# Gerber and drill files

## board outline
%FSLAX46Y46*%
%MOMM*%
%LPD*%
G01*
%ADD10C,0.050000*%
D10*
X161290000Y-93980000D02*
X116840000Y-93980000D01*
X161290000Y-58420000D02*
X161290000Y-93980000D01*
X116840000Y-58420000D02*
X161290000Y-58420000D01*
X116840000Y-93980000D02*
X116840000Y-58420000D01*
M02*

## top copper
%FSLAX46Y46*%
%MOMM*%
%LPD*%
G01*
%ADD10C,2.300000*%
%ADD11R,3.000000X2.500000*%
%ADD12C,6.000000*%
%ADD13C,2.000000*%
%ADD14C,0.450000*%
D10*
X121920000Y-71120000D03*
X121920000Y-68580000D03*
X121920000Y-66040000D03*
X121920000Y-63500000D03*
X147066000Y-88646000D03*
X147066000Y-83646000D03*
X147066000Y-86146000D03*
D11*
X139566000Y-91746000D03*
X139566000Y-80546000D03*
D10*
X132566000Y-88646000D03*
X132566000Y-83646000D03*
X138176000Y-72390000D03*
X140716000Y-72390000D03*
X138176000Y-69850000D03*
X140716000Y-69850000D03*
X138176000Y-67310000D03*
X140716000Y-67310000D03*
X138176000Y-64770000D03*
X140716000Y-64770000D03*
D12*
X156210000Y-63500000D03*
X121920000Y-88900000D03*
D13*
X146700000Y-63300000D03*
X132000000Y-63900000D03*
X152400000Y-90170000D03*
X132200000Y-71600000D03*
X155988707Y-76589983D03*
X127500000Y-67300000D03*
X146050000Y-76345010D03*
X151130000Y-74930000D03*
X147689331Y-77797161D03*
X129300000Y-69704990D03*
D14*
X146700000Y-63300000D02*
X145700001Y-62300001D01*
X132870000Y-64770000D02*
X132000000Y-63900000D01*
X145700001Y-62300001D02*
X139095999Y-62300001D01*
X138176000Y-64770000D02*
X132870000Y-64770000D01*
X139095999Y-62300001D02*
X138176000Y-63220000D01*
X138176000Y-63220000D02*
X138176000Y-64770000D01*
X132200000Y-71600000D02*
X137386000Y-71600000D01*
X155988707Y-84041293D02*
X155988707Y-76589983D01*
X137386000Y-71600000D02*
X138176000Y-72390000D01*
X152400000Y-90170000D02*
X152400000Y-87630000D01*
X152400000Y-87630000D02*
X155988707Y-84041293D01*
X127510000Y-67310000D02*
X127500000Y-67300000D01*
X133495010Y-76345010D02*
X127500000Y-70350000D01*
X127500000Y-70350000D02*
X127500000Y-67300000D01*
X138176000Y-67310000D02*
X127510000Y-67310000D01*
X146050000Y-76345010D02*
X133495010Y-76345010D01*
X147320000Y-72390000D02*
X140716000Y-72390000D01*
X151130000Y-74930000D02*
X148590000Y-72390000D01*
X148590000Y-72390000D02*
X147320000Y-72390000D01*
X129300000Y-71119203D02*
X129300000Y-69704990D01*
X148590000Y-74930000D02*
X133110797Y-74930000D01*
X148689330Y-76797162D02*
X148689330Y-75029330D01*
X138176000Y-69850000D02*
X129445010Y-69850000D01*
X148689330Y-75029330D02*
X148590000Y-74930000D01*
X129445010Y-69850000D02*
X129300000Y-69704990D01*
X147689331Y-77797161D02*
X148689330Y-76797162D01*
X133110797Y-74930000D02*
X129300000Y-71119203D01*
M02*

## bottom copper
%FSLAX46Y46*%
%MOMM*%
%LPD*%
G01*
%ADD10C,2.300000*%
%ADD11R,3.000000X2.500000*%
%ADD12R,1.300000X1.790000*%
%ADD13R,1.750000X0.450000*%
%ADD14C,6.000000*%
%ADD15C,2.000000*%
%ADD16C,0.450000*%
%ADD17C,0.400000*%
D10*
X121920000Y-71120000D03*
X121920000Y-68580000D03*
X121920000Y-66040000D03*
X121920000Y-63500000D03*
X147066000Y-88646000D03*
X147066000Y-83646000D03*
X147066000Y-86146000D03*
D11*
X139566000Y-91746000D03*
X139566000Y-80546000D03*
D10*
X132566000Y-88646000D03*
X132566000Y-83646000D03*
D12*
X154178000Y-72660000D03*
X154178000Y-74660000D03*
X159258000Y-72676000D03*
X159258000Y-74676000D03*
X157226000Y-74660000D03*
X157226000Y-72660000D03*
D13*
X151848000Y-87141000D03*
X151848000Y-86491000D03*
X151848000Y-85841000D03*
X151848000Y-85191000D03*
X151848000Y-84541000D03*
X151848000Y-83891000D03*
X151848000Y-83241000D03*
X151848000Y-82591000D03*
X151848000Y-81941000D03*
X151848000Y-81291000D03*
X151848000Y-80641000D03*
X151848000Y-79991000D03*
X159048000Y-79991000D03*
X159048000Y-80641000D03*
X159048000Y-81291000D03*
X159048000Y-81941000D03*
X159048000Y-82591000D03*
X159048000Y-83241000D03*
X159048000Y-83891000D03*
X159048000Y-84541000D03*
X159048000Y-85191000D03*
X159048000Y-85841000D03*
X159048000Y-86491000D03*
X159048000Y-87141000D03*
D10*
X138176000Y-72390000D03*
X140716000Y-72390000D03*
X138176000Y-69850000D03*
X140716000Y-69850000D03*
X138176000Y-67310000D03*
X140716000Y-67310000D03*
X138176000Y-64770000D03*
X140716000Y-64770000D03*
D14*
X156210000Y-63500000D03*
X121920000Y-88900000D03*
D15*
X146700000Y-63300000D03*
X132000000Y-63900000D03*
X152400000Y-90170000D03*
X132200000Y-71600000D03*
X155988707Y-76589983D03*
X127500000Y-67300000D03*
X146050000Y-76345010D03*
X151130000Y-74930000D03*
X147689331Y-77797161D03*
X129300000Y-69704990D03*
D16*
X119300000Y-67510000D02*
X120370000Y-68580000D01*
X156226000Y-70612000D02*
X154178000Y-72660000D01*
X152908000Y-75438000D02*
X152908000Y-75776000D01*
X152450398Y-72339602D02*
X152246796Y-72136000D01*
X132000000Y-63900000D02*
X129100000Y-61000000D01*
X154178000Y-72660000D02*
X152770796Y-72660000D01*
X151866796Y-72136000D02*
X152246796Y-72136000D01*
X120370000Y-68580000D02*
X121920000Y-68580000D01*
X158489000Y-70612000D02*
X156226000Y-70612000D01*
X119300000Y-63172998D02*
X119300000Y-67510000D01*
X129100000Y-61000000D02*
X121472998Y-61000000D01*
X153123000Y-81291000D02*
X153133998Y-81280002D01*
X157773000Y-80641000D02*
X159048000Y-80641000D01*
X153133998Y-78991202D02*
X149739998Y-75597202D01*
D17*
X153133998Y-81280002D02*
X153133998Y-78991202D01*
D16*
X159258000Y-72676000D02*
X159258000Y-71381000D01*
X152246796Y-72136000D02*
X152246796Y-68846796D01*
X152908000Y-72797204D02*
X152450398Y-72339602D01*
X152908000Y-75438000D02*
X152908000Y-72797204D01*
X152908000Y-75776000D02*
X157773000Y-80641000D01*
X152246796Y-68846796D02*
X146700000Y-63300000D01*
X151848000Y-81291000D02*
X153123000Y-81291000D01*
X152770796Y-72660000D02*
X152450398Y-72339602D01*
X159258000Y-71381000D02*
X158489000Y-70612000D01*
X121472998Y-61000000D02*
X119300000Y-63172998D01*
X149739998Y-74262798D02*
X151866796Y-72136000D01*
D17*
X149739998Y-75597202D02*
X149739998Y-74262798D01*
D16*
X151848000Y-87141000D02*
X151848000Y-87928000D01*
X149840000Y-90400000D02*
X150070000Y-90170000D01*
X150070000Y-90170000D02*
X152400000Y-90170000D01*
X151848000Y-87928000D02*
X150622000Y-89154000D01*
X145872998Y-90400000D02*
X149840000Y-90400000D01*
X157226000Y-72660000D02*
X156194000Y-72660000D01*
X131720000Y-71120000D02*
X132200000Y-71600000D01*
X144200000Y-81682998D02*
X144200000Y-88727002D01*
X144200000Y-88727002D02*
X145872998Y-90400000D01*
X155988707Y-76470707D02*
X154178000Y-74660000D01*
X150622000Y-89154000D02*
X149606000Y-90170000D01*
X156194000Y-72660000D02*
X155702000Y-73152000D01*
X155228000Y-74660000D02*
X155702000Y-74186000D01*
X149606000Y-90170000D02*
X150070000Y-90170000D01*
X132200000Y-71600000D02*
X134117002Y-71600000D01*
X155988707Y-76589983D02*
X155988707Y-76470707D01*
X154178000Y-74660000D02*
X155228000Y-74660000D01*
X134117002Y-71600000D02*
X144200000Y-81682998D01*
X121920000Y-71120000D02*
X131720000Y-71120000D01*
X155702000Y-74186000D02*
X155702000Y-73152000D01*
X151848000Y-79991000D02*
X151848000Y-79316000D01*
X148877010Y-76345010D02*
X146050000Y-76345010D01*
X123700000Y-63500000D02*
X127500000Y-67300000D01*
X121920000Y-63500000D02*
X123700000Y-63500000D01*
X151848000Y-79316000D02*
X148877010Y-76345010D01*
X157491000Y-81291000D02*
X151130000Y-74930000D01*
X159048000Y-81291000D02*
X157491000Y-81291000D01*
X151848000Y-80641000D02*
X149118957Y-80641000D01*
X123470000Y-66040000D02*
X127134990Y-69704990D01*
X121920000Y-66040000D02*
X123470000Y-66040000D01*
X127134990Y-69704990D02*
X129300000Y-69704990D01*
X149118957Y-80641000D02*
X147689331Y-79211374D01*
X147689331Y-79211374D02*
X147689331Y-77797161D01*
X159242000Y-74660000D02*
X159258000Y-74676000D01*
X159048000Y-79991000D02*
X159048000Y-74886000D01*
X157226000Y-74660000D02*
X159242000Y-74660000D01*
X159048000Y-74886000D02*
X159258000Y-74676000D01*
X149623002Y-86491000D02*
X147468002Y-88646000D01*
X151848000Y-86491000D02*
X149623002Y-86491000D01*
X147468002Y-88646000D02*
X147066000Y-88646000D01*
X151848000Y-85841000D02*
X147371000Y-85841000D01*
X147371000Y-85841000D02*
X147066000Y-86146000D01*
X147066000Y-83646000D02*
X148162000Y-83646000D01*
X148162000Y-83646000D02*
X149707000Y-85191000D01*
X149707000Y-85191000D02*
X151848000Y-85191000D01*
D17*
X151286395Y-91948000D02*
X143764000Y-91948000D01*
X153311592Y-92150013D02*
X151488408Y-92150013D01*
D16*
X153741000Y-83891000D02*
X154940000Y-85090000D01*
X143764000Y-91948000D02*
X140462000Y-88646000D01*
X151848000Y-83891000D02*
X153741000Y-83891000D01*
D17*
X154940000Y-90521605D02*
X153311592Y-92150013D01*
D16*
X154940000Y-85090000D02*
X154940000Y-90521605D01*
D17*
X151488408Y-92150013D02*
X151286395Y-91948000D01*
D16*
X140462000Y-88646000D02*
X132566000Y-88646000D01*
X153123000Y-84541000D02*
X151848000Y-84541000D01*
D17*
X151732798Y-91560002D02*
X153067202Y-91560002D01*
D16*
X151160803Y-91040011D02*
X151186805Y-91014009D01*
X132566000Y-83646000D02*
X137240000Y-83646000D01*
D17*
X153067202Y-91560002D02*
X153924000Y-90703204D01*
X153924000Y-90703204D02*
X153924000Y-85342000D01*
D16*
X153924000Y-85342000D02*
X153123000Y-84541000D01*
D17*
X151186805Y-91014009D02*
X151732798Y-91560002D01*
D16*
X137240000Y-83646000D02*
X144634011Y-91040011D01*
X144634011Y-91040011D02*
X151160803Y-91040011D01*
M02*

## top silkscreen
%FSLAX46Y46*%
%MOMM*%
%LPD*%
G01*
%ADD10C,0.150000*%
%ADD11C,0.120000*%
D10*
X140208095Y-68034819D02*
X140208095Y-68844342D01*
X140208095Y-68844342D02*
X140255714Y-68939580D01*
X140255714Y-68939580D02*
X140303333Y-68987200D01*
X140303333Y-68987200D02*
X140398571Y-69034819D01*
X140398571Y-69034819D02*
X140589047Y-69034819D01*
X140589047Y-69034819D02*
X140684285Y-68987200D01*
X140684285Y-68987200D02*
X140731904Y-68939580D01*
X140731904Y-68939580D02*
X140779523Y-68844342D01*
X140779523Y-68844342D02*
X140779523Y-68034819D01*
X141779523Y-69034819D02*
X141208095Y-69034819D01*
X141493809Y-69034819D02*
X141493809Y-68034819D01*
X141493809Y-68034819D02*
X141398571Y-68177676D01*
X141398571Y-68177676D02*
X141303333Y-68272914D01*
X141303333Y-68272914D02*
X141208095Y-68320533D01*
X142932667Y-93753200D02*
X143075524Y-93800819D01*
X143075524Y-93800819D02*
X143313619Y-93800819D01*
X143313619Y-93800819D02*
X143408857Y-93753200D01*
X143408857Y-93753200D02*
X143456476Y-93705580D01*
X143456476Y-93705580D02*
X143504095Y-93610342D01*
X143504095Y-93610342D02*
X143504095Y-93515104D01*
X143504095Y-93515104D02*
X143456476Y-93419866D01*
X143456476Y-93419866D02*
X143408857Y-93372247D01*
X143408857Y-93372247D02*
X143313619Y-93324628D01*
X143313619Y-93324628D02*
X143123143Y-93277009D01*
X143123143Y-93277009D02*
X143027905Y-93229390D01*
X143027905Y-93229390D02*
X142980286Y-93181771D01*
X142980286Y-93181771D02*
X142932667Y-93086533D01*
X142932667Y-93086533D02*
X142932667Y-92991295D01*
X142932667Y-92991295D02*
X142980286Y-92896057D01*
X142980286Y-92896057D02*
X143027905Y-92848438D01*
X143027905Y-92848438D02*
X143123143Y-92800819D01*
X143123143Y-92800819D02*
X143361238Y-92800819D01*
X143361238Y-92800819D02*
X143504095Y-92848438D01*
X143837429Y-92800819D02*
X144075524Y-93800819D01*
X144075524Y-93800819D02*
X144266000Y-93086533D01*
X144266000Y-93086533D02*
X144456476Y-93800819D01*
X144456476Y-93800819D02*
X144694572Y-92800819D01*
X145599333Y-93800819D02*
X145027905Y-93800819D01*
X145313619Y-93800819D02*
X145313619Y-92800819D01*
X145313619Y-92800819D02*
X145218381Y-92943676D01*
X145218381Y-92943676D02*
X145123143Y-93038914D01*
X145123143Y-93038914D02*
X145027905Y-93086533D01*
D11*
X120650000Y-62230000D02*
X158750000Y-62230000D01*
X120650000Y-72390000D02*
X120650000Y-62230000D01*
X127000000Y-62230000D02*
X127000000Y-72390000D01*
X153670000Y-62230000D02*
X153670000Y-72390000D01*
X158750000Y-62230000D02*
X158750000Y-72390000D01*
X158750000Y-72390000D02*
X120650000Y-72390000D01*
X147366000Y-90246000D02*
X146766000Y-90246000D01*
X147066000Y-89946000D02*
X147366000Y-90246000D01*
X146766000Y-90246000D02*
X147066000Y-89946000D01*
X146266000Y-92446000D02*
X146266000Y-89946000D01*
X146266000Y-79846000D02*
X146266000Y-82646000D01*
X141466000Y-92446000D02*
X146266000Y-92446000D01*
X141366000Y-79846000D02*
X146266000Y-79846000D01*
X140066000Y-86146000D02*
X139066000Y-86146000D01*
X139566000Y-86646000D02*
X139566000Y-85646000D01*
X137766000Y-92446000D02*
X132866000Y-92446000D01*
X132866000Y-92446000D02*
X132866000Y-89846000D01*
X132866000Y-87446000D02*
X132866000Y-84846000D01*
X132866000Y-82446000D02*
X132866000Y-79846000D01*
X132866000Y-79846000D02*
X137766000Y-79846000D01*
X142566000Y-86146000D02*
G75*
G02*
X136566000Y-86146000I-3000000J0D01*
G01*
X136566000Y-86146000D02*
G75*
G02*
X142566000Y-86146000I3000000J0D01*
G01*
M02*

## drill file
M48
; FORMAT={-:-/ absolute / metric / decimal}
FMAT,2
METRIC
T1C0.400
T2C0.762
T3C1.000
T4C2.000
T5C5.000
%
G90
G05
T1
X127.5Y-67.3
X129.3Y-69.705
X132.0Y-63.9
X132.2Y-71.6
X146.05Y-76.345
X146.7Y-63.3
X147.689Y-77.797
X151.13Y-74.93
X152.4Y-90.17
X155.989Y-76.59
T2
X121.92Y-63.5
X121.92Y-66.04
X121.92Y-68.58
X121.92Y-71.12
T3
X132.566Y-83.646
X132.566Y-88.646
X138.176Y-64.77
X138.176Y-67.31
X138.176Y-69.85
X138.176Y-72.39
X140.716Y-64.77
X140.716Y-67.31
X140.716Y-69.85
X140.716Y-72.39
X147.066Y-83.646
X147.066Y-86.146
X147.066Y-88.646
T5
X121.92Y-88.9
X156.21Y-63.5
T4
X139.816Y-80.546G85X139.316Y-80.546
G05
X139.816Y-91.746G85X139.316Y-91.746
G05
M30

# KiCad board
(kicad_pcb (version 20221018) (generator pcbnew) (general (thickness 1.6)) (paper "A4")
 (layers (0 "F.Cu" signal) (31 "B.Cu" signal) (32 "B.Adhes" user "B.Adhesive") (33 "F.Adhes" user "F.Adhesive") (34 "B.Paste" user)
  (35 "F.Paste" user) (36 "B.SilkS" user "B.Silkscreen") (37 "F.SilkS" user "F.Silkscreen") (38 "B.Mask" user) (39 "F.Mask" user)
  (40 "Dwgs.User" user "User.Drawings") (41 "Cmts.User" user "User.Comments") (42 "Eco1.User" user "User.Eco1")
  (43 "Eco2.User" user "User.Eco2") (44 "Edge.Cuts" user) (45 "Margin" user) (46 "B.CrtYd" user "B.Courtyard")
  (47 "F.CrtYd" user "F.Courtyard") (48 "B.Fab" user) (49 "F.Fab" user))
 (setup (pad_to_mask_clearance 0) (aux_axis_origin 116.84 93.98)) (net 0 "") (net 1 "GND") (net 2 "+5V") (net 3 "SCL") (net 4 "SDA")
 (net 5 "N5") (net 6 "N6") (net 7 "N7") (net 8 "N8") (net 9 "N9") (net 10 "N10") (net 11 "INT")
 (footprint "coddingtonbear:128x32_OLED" (layer "F.Cu") (at 129.54 68.58)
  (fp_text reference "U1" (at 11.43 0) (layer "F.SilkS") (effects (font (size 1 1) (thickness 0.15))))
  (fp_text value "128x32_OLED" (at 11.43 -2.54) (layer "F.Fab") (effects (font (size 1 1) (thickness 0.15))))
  (fp_line (start -8.89 -6.35) (end 29.21 -6.35) (stroke (width 0.12) (type solid)) (layer "F.SilkS"))
  (fp_line (start -8.89 3.81) (end -8.89 -6.35) (stroke (width 0.12) (type solid)) (layer "F.SilkS"))
  (fp_line (start -2.54 -6.35) (end -2.54 3.81) (stroke (width 0.12) (type solid)) (layer "F.SilkS"))
  (fp_line (start 24.13 -6.35) (end 24.13 3.81) (stroke (width 0.12) (type solid)) (layer "F.SilkS"))
  (fp_line (start 29.21 -6.35) (end 29.21 3.81) (stroke (width 0.12) (type solid)) (layer "F.SilkS"))
  (fp_line (start 29.21 3.81) (end -8.89 3.81) (stroke (width 0.12) (type solid)) (layer "F.SilkS"))
  (pad "1" thru_hole circle (at -7.62 2.54) (size 2.3 2.3) (drill 0.762) (layers "*.Cu" "*.Mask") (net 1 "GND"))
  (pad "2" thru_hole circle (at -7.62 0) (size 2.3 2.3) (drill 0.762) (layers "*.Cu" "*.Mask") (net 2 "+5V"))
  (pad "3" thru_hole circle (at -7.62 -2.54) (size 2.3 2.3) (drill 0.762) (layers "*.Cu" "*.Mask") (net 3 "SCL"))
  (pad "4" thru_hole circle (at -7.62 -5.08) (size 2.3 2.3) (drill 0.762) (layers "*.Cu" "*.Mask") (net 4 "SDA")))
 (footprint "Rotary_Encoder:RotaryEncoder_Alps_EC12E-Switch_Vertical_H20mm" (layer "F.Cu") (at 147.066 88.646 180)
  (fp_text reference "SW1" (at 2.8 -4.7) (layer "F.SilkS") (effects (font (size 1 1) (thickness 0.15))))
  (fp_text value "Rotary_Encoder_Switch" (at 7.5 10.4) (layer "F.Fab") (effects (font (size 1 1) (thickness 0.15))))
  (fp_line (start -0.3 -1.6) (end 0.3 -1.6) (stroke (width 0.12) (type solid)) (layer "F.SilkS"))
  (fp_line (start 0 -1.3) (end -0.3 -1.6) (stroke (width 0.12) (type solid)) (layer "F.SilkS"))
  (fp_line (start 0.3 -1.6) (end 0 -1.3) (stroke (width 0.12) (type solid)) (layer "F.SilkS"))
  (fp_line (start 0.8 -3.8) (end 0.8 -1.3) (stroke (width 0.12) (type solid)) (layer "F.SilkS"))
  (fp_line (start 0.8 8.8) (end 0.8 6) (stroke (width 0.12) (type solid)) (layer "F.SilkS"))
  (fp_line (start 5.6 -3.8) (end 0.8 -3.8) (stroke (width 0.12) (type solid)) (layer "F.SilkS"))
  (fp_line (start 5.7 8.8) (end 0.8 8.8) (stroke (width 0.12) (type solid)) (layer "F.SilkS"))
  (fp_line (start 7 2.5) (end 8 2.5) (stroke (width 0.12) (type solid)) (layer "F.SilkS"))
  (fp_line (start 7.5 2) (end 7.5 3) (stroke (width 0.12) (type solid)) (layer "F.SilkS"))
  (fp_line (start 9.3 -3.8) (end 14.2 -3.8) (stroke (width 0.12) (type solid)) (layer "F.SilkS"))
  (fp_line (start 14.2 -3.8) (end 14.2 -1.2) (stroke (width 0.12) (type solid)) (layer "F.SilkS"))
  (fp_line (start 14.2 1.2) (end 14.2 3.8) (stroke (width 0.12) (type solid)) (layer "F.SilkS"))
  (fp_line (start 14.2 6.2) (end 14.2 8.8) (stroke (width 0.12) (type solid)) (layer "F.SilkS"))
  (fp_line (start 14.2 8.8) (end 9.3 8.8) (stroke (width 0.12) (type solid)) (layer "F.SilkS"))
  (fp_circle (center 7.5 2.5) (end 10.5 2.5) (stroke (width 0.12) (type solid)) (fill none) (layer "F.SilkS"))
  (pad "A" thru_hole circle (at 0 0 180) (size 2.3 2.3) (drill 1) (layers "*.Cu" "*.Mask") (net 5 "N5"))
  (pad "B" thru_hole circle (at 0 5 180) (size 2.3 2.3) (drill 1) (layers "*.Cu" "*.Mask") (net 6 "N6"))
  (pad "C" thru_hole circle (at 0 2.5 180) (size 2.3 2.3) (drill 1) (layers "*.Cu" "*.Mask") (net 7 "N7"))
  (pad "MP" thru_hole rect (at 7.5 -3.1 180) (size 3 2.5) (drill oval 2.5 2) (layers "*.Cu" "*.Mask"))
  (pad "MP" thru_hole rect (at 7.5 8.1 180) (size 3 2.5) (drill oval 2.5 2) (layers "*.Cu" "*.Mask"))
  (pad "S1" thru_hole circle (at 14.5 0 180) (size 2.3 2.3) (drill 1) (layers "*.Cu" "*.Mask") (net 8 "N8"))
  (pad "S2" thru_hole circle (at 14.5 5 180) (size 2.3 2.3) (drill 1) (layers "*.Cu" "*.Mask") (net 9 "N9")))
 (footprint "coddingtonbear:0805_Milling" (layer "B.Cu") (at 154.178 73.66 -90)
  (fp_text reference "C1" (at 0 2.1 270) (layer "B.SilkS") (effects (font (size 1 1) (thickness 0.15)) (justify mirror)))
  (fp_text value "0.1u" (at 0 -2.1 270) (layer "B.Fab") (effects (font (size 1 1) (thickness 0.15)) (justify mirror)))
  (pad "1" smd rect (at -1 0 270) (size 1.79 1.3) (layers "B.Cu" "B.Paste" "B.Mask") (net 2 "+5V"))
  (pad "2" smd rect (at 1 0 270) (size 1.79 1.3) (layers "B.Cu" "B.Paste" "B.Mask") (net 1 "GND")))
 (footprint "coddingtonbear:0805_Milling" (layer "B.Cu") (at 159.258 73.676 -90)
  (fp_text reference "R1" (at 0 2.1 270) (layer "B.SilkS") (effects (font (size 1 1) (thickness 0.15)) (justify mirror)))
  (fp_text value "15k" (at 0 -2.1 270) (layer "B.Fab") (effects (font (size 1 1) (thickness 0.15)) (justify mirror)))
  (pad "1" smd rect (at -1 0 270) (size 1.79 1.3) (layers "B.Cu" "B.Paste" "B.Mask") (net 2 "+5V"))
  (pad "2" smd rect (at 1 0 270) (size 1.79 1.3) (layers "B.Cu" "B.Paste" "B.Mask") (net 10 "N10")))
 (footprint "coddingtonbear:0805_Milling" (layer "B.Cu") (at 157.226 73.66 90)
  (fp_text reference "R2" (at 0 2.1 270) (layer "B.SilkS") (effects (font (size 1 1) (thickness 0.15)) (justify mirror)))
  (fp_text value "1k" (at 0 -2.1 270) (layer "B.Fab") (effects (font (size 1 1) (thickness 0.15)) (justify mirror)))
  (pad "1" smd rect (at -1 0 90) (size 1.79 1.3) (layers "B.Cu" "B.Paste" "B.Mask") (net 10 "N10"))
  (pad "2" smd rect (at 1 0 90) (size 1.79 1.3) (layers "B.Cu" "B.Paste" "B.Mask") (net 1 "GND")))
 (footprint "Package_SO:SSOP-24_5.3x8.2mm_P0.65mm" (layer "B.Cu") (at 155.448 83.566)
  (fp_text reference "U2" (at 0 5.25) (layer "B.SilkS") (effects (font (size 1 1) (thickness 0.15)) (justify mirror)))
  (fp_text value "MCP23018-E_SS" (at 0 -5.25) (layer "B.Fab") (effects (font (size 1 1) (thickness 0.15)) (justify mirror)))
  (pad "1" smd rect (at -3.6 3.575) (size 1.75 0.45) (layers "B.Cu" "B.Paste" "B.Mask") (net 1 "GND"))
  (pad "2" smd rect (at -3.6 2.925) (size 1.75 0.45) (layers "B.Cu" "B.Paste" "B.Mask") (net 5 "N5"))
  (pad "3" smd rect (at -3.6 2.275) (size 1.75 0.45) (layers "B.Cu" "B.Paste" "B.Mask") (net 7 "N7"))
  (pad "4" smd rect (at -3.6 1.625) (size 1.75 0.45) (layers "B.Cu" "B.Paste" "B.Mask") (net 6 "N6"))
  (pad "5" smd rect (at -3.6 0.975) (size 1.75 0.45) (layers "B.Cu" "B.Paste" "B.Mask") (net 9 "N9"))
  (pad "6" smd rect (at -3.6 0.325) (size 1.75 0.45) (layers "B.Cu" "B.Paste" "B.Mask") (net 8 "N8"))
  (pad "7" smd rect (at -3.6 -0.325) (size 1.75 0.45) (layers "B.Cu" "B.Paste" "B.Mask"))
  (pad "8" smd rect (at -3.6 -0.975) (size 1.75 0.45) (layers "B.Cu" "B.Paste" "B.Mask"))
  (pad "9" smd rect (at -3.6 -1.625) (size 1.75 0.45) (layers "B.Cu" "B.Paste" "B.Mask"))
  (pad "10" smd rect (at -3.6 -2.275) (size 1.75 0.45) (layers "B.Cu" "B.Paste" "B.Mask") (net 2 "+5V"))
  (pad "11" smd rect (at -3.6 -2.925) (size 1.75 0.45) (layers "B.Cu" "B.Paste" "B.Mask") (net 3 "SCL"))
  (pad "12" smd rect (at -3.6 -3.575) (size 1.75 0.45) (layers "B.Cu" "B.Paste" "B.Mask") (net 4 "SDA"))
  (pad "13" smd rect (at 3.6 -3.575) (size 1.75 0.45) (layers "B.Cu" "B.Paste" "B.Mask") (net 10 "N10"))
  (pad "14" smd rect (at 3.6 -2.925) (size 1.75 0.45) (layers "B.Cu" "B.Paste" "B.Mask") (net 2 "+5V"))
  (pad "15" smd rect (at 3.6 -2.275) (size 1.75 0.45) (layers "B.Cu" "B.Paste" "B.Mask") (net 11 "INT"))
  (pad "16" smd rect (at 3.6 -1.625) (size 1.75 0.45) (layers "B.Cu" "B.Paste" "B.Mask"))
  (pad "17" smd rect (at 3.6 -0.975) (size 1.75 0.45) (layers "B.Cu" "B.Paste" "B.Mask"))
  (pad "18" smd rect (at 3.6 -0.325) (size 1.75 0.45) (layers "B.Cu" "B.Paste" "B.Mask"))
  (pad "19" smd rect (at 3.6 0.325) (size 1.75 0.45) (layers "B.Cu" "B.Paste" "B.Mask"))
  (pad "20" smd rect (at 3.6 0.975) (size 1.75 0.45) (layers "B.Cu" "B.Paste" "B.Mask"))
  (pad "21" smd rect (at 3.6 1.625) (size 1.75 0.45) (layers "B.Cu" "B.Paste" "B.Mask"))
  (pad "22" smd rect (at 3.6 2.275) (size 1.75 0.45) (layers "B.Cu" "B.Paste" "B.Mask"))
  (pad "23" smd rect (at 3.6 2.925) (size 1.75 0.45) (layers "B.Cu" "B.Paste" "B.Mask"))
  (pad "24" smd rect (at 3.6 3.575) (size 1.75 0.45) (layers "B.Cu" "B.Paste" "B.Mask")))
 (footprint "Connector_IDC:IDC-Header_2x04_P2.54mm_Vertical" (layer "B.Cu") (at 138.176 72.39)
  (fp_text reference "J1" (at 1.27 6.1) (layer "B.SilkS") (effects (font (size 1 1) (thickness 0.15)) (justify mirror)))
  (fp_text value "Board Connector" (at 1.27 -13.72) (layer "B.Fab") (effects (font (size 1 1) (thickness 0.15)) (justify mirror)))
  (pad "1" thru_hole circle (at 0 0) (size 2.3 2.3) (drill 1) (layers "*.Cu" "*.Mask") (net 1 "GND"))
  (pad "2" thru_hole circle (at 2.54 0) (size 2.3 2.3) (drill 1) (layers "*.Cu" "*.Mask") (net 11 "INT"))
  (pad "3" thru_hole circle (at 0 -2.54) (size 2.3 2.3) (drill 1) (layers "*.Cu" "*.Mask") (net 3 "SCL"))
  (pad "4" thru_hole circle (at 2.54 -2.54) (size 2.3 2.3) (drill 1) (layers "*.Cu" "*.Mask"))
  (pad "5" thru_hole circle (at 0 -5.08) (size 2.3 2.3) (drill 1) (layers "*.Cu" "*.Mask") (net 4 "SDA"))
  (pad "6" thru_hole circle (at 2.54 -5.08) (size 2.3 2.3) (drill 1) (layers "*.Cu" "*.Mask"))
  (pad "7" thru_hole circle (at 0 -7.62) (size 2.3 2.3) (drill 1) (layers "*.Cu" "*.Mask") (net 2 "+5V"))
  (pad "8" thru_hole circle (at 2.54 -7.62) (size 2.3 2.3) (drill 1) (layers "*.Cu" "*.Mask")))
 (gr_line (start 161.29 93.98) (end 116.84 93.98) (stroke (width 0.05) (type solid)) (layer "Edge.Cuts"))
 (gr_line (start 161.29 58.42) (end 161.29 93.98) (stroke (width 0.05) (type solid)) (layer "Edge.Cuts"))
 (gr_line (start 116.84 58.42) (end 161.29 58.42) (stroke (width 0.05) (type solid)) (layer "Edge.Cuts"))
 (gr_line (start 116.84 93.98) (end 116.84 58.42) (stroke (width 0.05) (type solid)) (layer "Edge.Cuts"))
 (via (at 156.21 63.5) (size 6) (drill 5) (layers "F.Cu" "B.Cu") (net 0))
 (via (at 121.92 88.9) (size 6) (drill 5) (layers "F.Cu" "B.Cu") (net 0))
 (segment (start 146.7 63.3) (end 145.700001 62.300001) (width 0.45) (layer "F.Cu") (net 2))
 (segment (start 132.87 64.77) (end 132 63.9) (width 0.45) (layer "F.Cu") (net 2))
 (segment (start 145.700001 62.300001) (end 139.095999 62.300001) (width 0.45) (layer "F.Cu") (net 2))
 (segment (start 138.176 64.77) (end 132.87 64.77) (width 0.45) (layer "F.Cu") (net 2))
 (segment (start 139.095999 62.300001) (end 138.176 63.22) (width 0.45) (layer "F.Cu") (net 2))
 (segment (start 138.176 63.22) (end 138.176 64.77) (width 0.45) (layer "F.Cu") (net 2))
 (via (at 146.7 63.3) (size 2) (drill 0.4) (layers "F.Cu" "B.Cu") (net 2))
 (via (at 132 63.9) (size 2) (drill 0.4) (layers "F.Cu" "B.Cu") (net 2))
 (segment (start 119.3 67.51) (end 120.37 68.58) (width 0.45) (layer "B.Cu") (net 2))
 (segment (start 156.226 70.612) (end 154.178 72.66) (width 0.45) (layer "B.Cu") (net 2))
 (segment (start 152.908 75.438) (end 152.908 75.776) (width 0.45) (layer "B.Cu") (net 2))
 (segment (start 152.450398 72.339602) (end 152.246796 72.136) (width 0.45) (layer "B.Cu") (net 2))
 (segment (start 132 63.9) (end 129.1 61) (width 0.45) (layer "B.Cu") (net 2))
 (segment (start 154.178 72.66) (end 152.770796 72.66) (width 0.45) (layer "B.Cu") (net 2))
 (segment (start 151.866796 72.136) (end 152.246796 72.136) (width 0.45) (layer "B.Cu") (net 2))
 (segment (start 120.37 68.58) (end 121.92 68.58) (width 0.45) (layer "B.Cu") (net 2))
 (segment (start 158.489 70.612) (end 156.226 70.612) (width 0.45) (layer "B.Cu") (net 2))
 (segment (start 119.3 63.172998) (end 119.3 67.51) (width 0.45) (layer "B.Cu") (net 2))
 (segment (start 129.1 61) (end 121.472998 61) (width 0.45) (layer "B.Cu") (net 2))
 (segment (start 153.123 81.291) (end 153.133998 81.280002) (width 0.45) (layer "B.Cu") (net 2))
 (segment (start 157.773 80.641) (end 159.048 80.641) (width 0.45) (layer "B.Cu") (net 2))
 (segment (start 153.133998 78.991202) (end 149.739998 75.597202) (width 0.45) (layer "B.Cu") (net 2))
 (segment (start 153.133998 81.280002) (end 153.133998 78.991202) (width 0.4) (layer "B.Cu") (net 2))
 (segment (start 159.258 72.676) (end 159.258 71.381) (width 0.45) (layer "B.Cu") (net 2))
 (segment (start 152.246796 72.136) (end 152.246796 68.846796) (width 0.45) (layer "B.Cu") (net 2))
 (segment (start 152.908 72.797204) (end 152.450398 72.339602) (width 0.45) (layer "B.Cu") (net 2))
 (segment (start 152.908 75.438) (end 152.908 72.797204) (width 0.45) (layer "B.Cu") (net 2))
 (segment (start 152.908 75.776) (end 157.773 80.641) (width 0.45) (layer "B.Cu") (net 2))
 (segment (start 152.246796 68.846796) (end 146.7 63.3) (width 0.45) (layer "B.Cu") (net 2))
 (segment (start 151.848 81.291) (end 153.123 81.291) (width 0.45) (layer "B.Cu") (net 2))
 (segment (start 152.770796 72.66) (end 152.450398 72.339602) (width 0.45) (layer "B.Cu") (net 2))
 (segment (start 159.258 71.381) (end 158.489 70.612) (width 0.45) (layer "B.Cu") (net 2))
 (segment (start 121.472998 61) (end 119.3 63.172998) (width 0.45) (layer "B.Cu") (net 2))
 (segment (start 149.739998 74.262798) (end 151.866796 72.136) (width 0.45) (layer "B.Cu") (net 2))
 (segment (start 149.739998 75.597202) (end 149.739998 74.262798) (width 0.4) (layer "B.Cu") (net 2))
 (segment (start 132.2 71.6) (end 137.386 71.6) (width 0.45) (layer "F.Cu") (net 1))
 (segment (start 155.988707 84.041293) (end 155.988707 76.589983) (width 0.45) (layer "F.Cu") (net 1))
 (segment (start 137.386 71.6) (end 138.176 72.39) (width 0.45) (layer "F.Cu") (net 1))
 (segment (start 152.4 90.17) (end 152.4 87.63) (width 0.45) (layer "F.Cu") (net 1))
 (segment (start 152.4 87.63) (end 155.988707 84.041293) (width 0.45) (layer "F.Cu") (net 1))
 (via (at 152.4 90.17) (size 2) (drill 0.4) (layers "F.Cu" "B.Cu") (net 1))
 (via (at 132.2 71.6) (size 2) (drill 0.4) (layers "F.Cu" "B.Cu") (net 1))
 (via (at 155.988707 76.589983) (size 2) (drill 0.4) (layers "F.Cu" "B.Cu") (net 1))
 (segment (start 151.848 87.141) (end 151.848 87.928) (width 0.45) (layer "B.Cu") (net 1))
 (segment (start 149.84 90.4) (end 150.07 90.17) (width 0.45) (layer "B.Cu") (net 1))
 (segment (start 150.07 90.17) (end 152.4 90.17) (width 0.45) (layer "B.Cu") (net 1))
 (segment (start 151.848 87.928) (end 150.622 89.154) (width 0.45) (layer "B.Cu") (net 1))
 (segment (start 145.872998 90.4) (end 149.84 90.4) (width 0.45) (layer "B.Cu") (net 1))
 (segment (start 157.226 72.66) (end 156.194 72.66) (width 0.45) (layer "B.Cu") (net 1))
 (segment (start 131.72 71.12) (end 132.2 71.6) (width 0.45) (layer "B.Cu") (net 1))
 (segment (start 144.2 81.682998) (end 144.2 88.727002) (width 0.45) (layer "B.Cu") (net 1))
 (segment (start 144.2 88.727002) (end 145.872998 90.4) (width 0.45) (layer "B.Cu") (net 1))
 (segment (start 155.988707 76.470707) (end 154.178 74.66) (width 0.45) (layer "B.Cu") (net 1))
 (segment (start 150.622 89.154) (end 149.606 90.17) (width 0.45) (layer "B.Cu") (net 1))
 (segment (start 156.194 72.66) (end 155.702 73.152) (width 0.45) (layer "B.Cu") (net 1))
 (segment (start 155.228 74.66) (end 155.702 74.186) (width 0.45) (layer "B.Cu") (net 1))
 (segment (start 149.606 90.17) (end 150.07 90.17) (width 0.45) (layer "B.Cu") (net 1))
 (segment (start 132.2 71.6) (end 134.117002 71.6) (width 0.45) (layer "B.Cu") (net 1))
 (segment (start 155.988707 76.589983) (end 155.988707 76.470707) (width 0.45) (layer "B.Cu") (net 1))
 (segment (start 154.178 74.66) (end 155.228 74.66) (width 0.45) (layer "B.Cu") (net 1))
 (segment (start 134.117002 71.6) (end 144.2 81.682998) (width 0.45) (layer "B.Cu") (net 1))
 (segment (start 121.92 71.12) (end 131.72 71.12) (width 0.45) (layer "B.Cu") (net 1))
 (segment (start 155.702 74.186) (end 155.702 73.152) (width 0.45) (layer "B.Cu") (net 1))
 (segment (start 127.51 67.31) (end 127.5 67.3) (width 0.45) (layer "F.Cu") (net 4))
 (segment (start 133.49501 76.34501) (end 127.5 70.35) (width 0.45) (layer "F.Cu") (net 4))
 (segment (start 127.5 70.35) (end 127.5 67.3) (width 0.45) (layer "F.Cu") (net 4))
 (segment (start 138.176 67.31) (end 127.51 67.31) (width 0.45) (layer "F.Cu") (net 4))
 (segment (start 146.05 76.34501) (end 133.49501 76.34501) (width 0.45) (layer "F.Cu") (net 4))
 (via (at 127.5 67.3) (size 2) (drill 0.4) (layers "F.Cu" "B.Cu") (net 4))
 (via (at 146.05 76.34501) (size 2) (drill 0.4) (layers "F.Cu" "B.Cu") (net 4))
 (segment (start 151.848 79.991) (end 151.848 79.316) (width 0.45) (layer "B.Cu") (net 4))
 (segment (start 148.87701 76.34501) (end 146.05 76.34501) (width 0.45) (layer "B.Cu") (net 4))
 (segment (start 123.7 63.5) (end 127.5 67.3) (width 0.45) (layer "B.Cu") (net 4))
 (segment (start 121.92 63.5) (end 123.7 63.5) (width 0.45) (layer "B.Cu") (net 4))
 (segment (start 151.848 79.316) (end 148.87701 76.34501) (width 0.45) (layer "B.Cu") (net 4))
 (segment (start 147.32 72.39) (end 140.716 72.39) (width 0.45) (layer "F.Cu") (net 11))
 (segment (start 151.13 74.93) (end 148.59 72.39) (width 0.45) (layer "F.Cu") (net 11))
 (segment (start 148.59 72.39) (end 147.32 72.39) (width 0.45) (layer "F.Cu") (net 11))
 (via (at 151.13 74.93) (size 2) (drill 0.4) (layers "F.Cu" "B.Cu") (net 11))
 (segment (start 157.491 81.291) (end 151.13 74.93) (width 0.45) (layer "B.Cu") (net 11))
 (segment (start 159.048 81.291) (end 157.491 81.291) (width 0.45) (layer "B.Cu") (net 11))
 (segment (start 129.3 71.119203) (end 129.3 69.70499) (width 0.45) (layer "F.Cu") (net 3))
 (segment (start 148.59 74.93) (end 133.110797 74.93) (width 0.45) (layer "F.Cu") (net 3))
 (segment (start 148.68933 76.797162) (end 148.68933 75.02933) (width 0.45) (layer "F.Cu") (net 3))
 (segment (start 138.176 69.85) (end 129.44501 69.85) (width 0.45) (layer "F.Cu") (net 3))
 (segment (start 148.68933 75.02933) (end 148.59 74.93) (width 0.45) (layer "F.Cu") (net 3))
 (segment (start 129.44501 69.85) (end 129.3 69.70499) (width 0.45) (layer "F.Cu") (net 3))
 (segment (start 147.689331 77.797161) (end 148.68933 76.797162) (width 0.45) (layer "F.Cu") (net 3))
 (segment (start 133.110797 74.93) (end 129.3 71.119203) (width 0.45) (layer "F.Cu") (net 3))
 (via (at 147.689331 77.797161) (size 2) (drill 0.4) (layers "F.Cu" "B.Cu") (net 3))
 (via (at 129.3 69.70499) (size 2) (drill 0.4) (layers "F.Cu" "B.Cu") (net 3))
 (segment (start 151.848 80.641) (end 149.118957 80.641) (width 0.45) (layer "B.Cu") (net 3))
 (segment (start 123.47 66.04) (end 127.13499 69.70499) (width 0.45) (layer "B.Cu") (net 3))
 (segment (start 121.92 66.04) (end 123.47 66.04) (width 0.45) (layer "B.Cu") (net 3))
 (segment (start 127.13499 69.70499) (end 129.3 69.70499) (width 0.45) (layer "B.Cu") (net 3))
 (segment (start 149.118957 80.641) (end 147.689331 79.211374) (width 0.45) (layer "B.Cu") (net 3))
 (segment (start 147.689331 79.211374) (end 147.689331 77.797161) (width 0.45) (layer "B.Cu") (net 3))
 (segment (start 159.242 74.66) (end 159.258 74.676) (width 0.45) (layer "B.Cu") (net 10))
 (segment (start 159.048 79.991) (end 159.048 74.886) (width 0.45) (layer "B.Cu") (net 10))
 (segment (start 157.226 74.66) (end 159.242 74.66) (width 0.45) (layer "B.Cu") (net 10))
 (segment (start 159.048 74.886) (end 159.258 74.676) (width 0.45) (layer "B.Cu") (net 10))
 (segment (start 149.623002 86.491) (end 147.468002 88.646) (width 0.45) (layer "B.Cu") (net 5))
 (segment (start 151.848 86.491) (end 149.623002 86.491) (width 0.45) (layer "B.Cu") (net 5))
 (segment (start 147.468002 88.646) (end 147.066 88.646) (width 0.45) (layer "B.Cu") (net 5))
 (segment (start 151.848 85.841) (end 147.371 85.841) (width 0.45) (layer "B.Cu") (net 7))
 (segment (start 147.371 85.841) (end 147.066 86.146) (width 0.45) (layer "B.Cu") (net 7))
 (segment (start 147.066 83.646) (end 148.162 83.646) (width 0.45) (layer "B.Cu") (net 6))
 (segment (start 148.162 83.646) (end 149.707 85.191) (width 0.45) (layer "B.Cu") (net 6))
 (segment (start 149.707 85.191) (end 151.848 85.191) (width 0.45) (layer "B.Cu") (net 6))
 (segment (start 151.286395 91.948) (end 143.764 91.948) (width 0.4) (layer "B.Cu") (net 8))
 (segment (start 153.311592 92.150013) (end 151.488408 92.150013) (width 0.4) (layer "B.Cu") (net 8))
 (segment (start 153.741 83.891) (end 154.94 85.09) (width 0.45) (layer "B.Cu") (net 8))
 (segment (start 143.764 91.948) (end 140.462 88.646) (width 0.45) (layer "B.Cu") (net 8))
 (segment (start 151.848 83.891) (end 153.741 83.891) (width 0.45) (layer "B.Cu") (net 8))
 (segment (start 154.94 90.521605) (end 153.311592 92.150013) (width 0.4) (layer "B.Cu") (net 8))
 (segment (start 154.94 85.09) (end 154.94 90.521605) (width 0.45) (layer "B.Cu") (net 8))
 (segment (start 151.488408 92.150013) (end 151.286395 91.948) (width 0.4) (layer "B.Cu") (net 8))
 (segment (start 140.462 88.646) (end 132.566 88.646) (width 0.45) (layer "B.Cu") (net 8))
 (segment (start 153.123 84.541) (end 151.848 84.541) (width 0.45) (layer "B.Cu") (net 9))
 (segment (start 151.732798 91.560002) (end 153.067202 91.560002) (width 0.4) (layer "B.Cu") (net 9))
 (segment (start 151.160803 91.040011) (end 151.186805 91.014009) (width 0.45) (layer "B.Cu") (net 9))
 (segment (start 132.566 83.646) (end 137.24 83.646) (width 0.45) (layer "B.Cu") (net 9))
 (segment (start 153.067202 91.560002) (end 153.924 90.703204) (width 0.4) (layer "B.Cu") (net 9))
 (segment (start 153.924 90.703204) (end 153.924 85.342) (width 0.4) (layer "B.Cu") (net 9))
 (segment (start 153.924 85.342) (end 153.123 84.541) (width 0.45) (layer "B.Cu") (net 9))
 (segment (start 151.186805 91.014009) (end 151.732798 91.560002) (width 0.4) (layer "B.Cu") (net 9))
 (segment (start 137.24 83.646) (end 144.634011 91.040011) (width 0.45) (layer "B.Cu") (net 9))
 (segment (start 144.634011 91.040011) (end 151.160803 91.040011) (width 0.45) (layer "B.Cu") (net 9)))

